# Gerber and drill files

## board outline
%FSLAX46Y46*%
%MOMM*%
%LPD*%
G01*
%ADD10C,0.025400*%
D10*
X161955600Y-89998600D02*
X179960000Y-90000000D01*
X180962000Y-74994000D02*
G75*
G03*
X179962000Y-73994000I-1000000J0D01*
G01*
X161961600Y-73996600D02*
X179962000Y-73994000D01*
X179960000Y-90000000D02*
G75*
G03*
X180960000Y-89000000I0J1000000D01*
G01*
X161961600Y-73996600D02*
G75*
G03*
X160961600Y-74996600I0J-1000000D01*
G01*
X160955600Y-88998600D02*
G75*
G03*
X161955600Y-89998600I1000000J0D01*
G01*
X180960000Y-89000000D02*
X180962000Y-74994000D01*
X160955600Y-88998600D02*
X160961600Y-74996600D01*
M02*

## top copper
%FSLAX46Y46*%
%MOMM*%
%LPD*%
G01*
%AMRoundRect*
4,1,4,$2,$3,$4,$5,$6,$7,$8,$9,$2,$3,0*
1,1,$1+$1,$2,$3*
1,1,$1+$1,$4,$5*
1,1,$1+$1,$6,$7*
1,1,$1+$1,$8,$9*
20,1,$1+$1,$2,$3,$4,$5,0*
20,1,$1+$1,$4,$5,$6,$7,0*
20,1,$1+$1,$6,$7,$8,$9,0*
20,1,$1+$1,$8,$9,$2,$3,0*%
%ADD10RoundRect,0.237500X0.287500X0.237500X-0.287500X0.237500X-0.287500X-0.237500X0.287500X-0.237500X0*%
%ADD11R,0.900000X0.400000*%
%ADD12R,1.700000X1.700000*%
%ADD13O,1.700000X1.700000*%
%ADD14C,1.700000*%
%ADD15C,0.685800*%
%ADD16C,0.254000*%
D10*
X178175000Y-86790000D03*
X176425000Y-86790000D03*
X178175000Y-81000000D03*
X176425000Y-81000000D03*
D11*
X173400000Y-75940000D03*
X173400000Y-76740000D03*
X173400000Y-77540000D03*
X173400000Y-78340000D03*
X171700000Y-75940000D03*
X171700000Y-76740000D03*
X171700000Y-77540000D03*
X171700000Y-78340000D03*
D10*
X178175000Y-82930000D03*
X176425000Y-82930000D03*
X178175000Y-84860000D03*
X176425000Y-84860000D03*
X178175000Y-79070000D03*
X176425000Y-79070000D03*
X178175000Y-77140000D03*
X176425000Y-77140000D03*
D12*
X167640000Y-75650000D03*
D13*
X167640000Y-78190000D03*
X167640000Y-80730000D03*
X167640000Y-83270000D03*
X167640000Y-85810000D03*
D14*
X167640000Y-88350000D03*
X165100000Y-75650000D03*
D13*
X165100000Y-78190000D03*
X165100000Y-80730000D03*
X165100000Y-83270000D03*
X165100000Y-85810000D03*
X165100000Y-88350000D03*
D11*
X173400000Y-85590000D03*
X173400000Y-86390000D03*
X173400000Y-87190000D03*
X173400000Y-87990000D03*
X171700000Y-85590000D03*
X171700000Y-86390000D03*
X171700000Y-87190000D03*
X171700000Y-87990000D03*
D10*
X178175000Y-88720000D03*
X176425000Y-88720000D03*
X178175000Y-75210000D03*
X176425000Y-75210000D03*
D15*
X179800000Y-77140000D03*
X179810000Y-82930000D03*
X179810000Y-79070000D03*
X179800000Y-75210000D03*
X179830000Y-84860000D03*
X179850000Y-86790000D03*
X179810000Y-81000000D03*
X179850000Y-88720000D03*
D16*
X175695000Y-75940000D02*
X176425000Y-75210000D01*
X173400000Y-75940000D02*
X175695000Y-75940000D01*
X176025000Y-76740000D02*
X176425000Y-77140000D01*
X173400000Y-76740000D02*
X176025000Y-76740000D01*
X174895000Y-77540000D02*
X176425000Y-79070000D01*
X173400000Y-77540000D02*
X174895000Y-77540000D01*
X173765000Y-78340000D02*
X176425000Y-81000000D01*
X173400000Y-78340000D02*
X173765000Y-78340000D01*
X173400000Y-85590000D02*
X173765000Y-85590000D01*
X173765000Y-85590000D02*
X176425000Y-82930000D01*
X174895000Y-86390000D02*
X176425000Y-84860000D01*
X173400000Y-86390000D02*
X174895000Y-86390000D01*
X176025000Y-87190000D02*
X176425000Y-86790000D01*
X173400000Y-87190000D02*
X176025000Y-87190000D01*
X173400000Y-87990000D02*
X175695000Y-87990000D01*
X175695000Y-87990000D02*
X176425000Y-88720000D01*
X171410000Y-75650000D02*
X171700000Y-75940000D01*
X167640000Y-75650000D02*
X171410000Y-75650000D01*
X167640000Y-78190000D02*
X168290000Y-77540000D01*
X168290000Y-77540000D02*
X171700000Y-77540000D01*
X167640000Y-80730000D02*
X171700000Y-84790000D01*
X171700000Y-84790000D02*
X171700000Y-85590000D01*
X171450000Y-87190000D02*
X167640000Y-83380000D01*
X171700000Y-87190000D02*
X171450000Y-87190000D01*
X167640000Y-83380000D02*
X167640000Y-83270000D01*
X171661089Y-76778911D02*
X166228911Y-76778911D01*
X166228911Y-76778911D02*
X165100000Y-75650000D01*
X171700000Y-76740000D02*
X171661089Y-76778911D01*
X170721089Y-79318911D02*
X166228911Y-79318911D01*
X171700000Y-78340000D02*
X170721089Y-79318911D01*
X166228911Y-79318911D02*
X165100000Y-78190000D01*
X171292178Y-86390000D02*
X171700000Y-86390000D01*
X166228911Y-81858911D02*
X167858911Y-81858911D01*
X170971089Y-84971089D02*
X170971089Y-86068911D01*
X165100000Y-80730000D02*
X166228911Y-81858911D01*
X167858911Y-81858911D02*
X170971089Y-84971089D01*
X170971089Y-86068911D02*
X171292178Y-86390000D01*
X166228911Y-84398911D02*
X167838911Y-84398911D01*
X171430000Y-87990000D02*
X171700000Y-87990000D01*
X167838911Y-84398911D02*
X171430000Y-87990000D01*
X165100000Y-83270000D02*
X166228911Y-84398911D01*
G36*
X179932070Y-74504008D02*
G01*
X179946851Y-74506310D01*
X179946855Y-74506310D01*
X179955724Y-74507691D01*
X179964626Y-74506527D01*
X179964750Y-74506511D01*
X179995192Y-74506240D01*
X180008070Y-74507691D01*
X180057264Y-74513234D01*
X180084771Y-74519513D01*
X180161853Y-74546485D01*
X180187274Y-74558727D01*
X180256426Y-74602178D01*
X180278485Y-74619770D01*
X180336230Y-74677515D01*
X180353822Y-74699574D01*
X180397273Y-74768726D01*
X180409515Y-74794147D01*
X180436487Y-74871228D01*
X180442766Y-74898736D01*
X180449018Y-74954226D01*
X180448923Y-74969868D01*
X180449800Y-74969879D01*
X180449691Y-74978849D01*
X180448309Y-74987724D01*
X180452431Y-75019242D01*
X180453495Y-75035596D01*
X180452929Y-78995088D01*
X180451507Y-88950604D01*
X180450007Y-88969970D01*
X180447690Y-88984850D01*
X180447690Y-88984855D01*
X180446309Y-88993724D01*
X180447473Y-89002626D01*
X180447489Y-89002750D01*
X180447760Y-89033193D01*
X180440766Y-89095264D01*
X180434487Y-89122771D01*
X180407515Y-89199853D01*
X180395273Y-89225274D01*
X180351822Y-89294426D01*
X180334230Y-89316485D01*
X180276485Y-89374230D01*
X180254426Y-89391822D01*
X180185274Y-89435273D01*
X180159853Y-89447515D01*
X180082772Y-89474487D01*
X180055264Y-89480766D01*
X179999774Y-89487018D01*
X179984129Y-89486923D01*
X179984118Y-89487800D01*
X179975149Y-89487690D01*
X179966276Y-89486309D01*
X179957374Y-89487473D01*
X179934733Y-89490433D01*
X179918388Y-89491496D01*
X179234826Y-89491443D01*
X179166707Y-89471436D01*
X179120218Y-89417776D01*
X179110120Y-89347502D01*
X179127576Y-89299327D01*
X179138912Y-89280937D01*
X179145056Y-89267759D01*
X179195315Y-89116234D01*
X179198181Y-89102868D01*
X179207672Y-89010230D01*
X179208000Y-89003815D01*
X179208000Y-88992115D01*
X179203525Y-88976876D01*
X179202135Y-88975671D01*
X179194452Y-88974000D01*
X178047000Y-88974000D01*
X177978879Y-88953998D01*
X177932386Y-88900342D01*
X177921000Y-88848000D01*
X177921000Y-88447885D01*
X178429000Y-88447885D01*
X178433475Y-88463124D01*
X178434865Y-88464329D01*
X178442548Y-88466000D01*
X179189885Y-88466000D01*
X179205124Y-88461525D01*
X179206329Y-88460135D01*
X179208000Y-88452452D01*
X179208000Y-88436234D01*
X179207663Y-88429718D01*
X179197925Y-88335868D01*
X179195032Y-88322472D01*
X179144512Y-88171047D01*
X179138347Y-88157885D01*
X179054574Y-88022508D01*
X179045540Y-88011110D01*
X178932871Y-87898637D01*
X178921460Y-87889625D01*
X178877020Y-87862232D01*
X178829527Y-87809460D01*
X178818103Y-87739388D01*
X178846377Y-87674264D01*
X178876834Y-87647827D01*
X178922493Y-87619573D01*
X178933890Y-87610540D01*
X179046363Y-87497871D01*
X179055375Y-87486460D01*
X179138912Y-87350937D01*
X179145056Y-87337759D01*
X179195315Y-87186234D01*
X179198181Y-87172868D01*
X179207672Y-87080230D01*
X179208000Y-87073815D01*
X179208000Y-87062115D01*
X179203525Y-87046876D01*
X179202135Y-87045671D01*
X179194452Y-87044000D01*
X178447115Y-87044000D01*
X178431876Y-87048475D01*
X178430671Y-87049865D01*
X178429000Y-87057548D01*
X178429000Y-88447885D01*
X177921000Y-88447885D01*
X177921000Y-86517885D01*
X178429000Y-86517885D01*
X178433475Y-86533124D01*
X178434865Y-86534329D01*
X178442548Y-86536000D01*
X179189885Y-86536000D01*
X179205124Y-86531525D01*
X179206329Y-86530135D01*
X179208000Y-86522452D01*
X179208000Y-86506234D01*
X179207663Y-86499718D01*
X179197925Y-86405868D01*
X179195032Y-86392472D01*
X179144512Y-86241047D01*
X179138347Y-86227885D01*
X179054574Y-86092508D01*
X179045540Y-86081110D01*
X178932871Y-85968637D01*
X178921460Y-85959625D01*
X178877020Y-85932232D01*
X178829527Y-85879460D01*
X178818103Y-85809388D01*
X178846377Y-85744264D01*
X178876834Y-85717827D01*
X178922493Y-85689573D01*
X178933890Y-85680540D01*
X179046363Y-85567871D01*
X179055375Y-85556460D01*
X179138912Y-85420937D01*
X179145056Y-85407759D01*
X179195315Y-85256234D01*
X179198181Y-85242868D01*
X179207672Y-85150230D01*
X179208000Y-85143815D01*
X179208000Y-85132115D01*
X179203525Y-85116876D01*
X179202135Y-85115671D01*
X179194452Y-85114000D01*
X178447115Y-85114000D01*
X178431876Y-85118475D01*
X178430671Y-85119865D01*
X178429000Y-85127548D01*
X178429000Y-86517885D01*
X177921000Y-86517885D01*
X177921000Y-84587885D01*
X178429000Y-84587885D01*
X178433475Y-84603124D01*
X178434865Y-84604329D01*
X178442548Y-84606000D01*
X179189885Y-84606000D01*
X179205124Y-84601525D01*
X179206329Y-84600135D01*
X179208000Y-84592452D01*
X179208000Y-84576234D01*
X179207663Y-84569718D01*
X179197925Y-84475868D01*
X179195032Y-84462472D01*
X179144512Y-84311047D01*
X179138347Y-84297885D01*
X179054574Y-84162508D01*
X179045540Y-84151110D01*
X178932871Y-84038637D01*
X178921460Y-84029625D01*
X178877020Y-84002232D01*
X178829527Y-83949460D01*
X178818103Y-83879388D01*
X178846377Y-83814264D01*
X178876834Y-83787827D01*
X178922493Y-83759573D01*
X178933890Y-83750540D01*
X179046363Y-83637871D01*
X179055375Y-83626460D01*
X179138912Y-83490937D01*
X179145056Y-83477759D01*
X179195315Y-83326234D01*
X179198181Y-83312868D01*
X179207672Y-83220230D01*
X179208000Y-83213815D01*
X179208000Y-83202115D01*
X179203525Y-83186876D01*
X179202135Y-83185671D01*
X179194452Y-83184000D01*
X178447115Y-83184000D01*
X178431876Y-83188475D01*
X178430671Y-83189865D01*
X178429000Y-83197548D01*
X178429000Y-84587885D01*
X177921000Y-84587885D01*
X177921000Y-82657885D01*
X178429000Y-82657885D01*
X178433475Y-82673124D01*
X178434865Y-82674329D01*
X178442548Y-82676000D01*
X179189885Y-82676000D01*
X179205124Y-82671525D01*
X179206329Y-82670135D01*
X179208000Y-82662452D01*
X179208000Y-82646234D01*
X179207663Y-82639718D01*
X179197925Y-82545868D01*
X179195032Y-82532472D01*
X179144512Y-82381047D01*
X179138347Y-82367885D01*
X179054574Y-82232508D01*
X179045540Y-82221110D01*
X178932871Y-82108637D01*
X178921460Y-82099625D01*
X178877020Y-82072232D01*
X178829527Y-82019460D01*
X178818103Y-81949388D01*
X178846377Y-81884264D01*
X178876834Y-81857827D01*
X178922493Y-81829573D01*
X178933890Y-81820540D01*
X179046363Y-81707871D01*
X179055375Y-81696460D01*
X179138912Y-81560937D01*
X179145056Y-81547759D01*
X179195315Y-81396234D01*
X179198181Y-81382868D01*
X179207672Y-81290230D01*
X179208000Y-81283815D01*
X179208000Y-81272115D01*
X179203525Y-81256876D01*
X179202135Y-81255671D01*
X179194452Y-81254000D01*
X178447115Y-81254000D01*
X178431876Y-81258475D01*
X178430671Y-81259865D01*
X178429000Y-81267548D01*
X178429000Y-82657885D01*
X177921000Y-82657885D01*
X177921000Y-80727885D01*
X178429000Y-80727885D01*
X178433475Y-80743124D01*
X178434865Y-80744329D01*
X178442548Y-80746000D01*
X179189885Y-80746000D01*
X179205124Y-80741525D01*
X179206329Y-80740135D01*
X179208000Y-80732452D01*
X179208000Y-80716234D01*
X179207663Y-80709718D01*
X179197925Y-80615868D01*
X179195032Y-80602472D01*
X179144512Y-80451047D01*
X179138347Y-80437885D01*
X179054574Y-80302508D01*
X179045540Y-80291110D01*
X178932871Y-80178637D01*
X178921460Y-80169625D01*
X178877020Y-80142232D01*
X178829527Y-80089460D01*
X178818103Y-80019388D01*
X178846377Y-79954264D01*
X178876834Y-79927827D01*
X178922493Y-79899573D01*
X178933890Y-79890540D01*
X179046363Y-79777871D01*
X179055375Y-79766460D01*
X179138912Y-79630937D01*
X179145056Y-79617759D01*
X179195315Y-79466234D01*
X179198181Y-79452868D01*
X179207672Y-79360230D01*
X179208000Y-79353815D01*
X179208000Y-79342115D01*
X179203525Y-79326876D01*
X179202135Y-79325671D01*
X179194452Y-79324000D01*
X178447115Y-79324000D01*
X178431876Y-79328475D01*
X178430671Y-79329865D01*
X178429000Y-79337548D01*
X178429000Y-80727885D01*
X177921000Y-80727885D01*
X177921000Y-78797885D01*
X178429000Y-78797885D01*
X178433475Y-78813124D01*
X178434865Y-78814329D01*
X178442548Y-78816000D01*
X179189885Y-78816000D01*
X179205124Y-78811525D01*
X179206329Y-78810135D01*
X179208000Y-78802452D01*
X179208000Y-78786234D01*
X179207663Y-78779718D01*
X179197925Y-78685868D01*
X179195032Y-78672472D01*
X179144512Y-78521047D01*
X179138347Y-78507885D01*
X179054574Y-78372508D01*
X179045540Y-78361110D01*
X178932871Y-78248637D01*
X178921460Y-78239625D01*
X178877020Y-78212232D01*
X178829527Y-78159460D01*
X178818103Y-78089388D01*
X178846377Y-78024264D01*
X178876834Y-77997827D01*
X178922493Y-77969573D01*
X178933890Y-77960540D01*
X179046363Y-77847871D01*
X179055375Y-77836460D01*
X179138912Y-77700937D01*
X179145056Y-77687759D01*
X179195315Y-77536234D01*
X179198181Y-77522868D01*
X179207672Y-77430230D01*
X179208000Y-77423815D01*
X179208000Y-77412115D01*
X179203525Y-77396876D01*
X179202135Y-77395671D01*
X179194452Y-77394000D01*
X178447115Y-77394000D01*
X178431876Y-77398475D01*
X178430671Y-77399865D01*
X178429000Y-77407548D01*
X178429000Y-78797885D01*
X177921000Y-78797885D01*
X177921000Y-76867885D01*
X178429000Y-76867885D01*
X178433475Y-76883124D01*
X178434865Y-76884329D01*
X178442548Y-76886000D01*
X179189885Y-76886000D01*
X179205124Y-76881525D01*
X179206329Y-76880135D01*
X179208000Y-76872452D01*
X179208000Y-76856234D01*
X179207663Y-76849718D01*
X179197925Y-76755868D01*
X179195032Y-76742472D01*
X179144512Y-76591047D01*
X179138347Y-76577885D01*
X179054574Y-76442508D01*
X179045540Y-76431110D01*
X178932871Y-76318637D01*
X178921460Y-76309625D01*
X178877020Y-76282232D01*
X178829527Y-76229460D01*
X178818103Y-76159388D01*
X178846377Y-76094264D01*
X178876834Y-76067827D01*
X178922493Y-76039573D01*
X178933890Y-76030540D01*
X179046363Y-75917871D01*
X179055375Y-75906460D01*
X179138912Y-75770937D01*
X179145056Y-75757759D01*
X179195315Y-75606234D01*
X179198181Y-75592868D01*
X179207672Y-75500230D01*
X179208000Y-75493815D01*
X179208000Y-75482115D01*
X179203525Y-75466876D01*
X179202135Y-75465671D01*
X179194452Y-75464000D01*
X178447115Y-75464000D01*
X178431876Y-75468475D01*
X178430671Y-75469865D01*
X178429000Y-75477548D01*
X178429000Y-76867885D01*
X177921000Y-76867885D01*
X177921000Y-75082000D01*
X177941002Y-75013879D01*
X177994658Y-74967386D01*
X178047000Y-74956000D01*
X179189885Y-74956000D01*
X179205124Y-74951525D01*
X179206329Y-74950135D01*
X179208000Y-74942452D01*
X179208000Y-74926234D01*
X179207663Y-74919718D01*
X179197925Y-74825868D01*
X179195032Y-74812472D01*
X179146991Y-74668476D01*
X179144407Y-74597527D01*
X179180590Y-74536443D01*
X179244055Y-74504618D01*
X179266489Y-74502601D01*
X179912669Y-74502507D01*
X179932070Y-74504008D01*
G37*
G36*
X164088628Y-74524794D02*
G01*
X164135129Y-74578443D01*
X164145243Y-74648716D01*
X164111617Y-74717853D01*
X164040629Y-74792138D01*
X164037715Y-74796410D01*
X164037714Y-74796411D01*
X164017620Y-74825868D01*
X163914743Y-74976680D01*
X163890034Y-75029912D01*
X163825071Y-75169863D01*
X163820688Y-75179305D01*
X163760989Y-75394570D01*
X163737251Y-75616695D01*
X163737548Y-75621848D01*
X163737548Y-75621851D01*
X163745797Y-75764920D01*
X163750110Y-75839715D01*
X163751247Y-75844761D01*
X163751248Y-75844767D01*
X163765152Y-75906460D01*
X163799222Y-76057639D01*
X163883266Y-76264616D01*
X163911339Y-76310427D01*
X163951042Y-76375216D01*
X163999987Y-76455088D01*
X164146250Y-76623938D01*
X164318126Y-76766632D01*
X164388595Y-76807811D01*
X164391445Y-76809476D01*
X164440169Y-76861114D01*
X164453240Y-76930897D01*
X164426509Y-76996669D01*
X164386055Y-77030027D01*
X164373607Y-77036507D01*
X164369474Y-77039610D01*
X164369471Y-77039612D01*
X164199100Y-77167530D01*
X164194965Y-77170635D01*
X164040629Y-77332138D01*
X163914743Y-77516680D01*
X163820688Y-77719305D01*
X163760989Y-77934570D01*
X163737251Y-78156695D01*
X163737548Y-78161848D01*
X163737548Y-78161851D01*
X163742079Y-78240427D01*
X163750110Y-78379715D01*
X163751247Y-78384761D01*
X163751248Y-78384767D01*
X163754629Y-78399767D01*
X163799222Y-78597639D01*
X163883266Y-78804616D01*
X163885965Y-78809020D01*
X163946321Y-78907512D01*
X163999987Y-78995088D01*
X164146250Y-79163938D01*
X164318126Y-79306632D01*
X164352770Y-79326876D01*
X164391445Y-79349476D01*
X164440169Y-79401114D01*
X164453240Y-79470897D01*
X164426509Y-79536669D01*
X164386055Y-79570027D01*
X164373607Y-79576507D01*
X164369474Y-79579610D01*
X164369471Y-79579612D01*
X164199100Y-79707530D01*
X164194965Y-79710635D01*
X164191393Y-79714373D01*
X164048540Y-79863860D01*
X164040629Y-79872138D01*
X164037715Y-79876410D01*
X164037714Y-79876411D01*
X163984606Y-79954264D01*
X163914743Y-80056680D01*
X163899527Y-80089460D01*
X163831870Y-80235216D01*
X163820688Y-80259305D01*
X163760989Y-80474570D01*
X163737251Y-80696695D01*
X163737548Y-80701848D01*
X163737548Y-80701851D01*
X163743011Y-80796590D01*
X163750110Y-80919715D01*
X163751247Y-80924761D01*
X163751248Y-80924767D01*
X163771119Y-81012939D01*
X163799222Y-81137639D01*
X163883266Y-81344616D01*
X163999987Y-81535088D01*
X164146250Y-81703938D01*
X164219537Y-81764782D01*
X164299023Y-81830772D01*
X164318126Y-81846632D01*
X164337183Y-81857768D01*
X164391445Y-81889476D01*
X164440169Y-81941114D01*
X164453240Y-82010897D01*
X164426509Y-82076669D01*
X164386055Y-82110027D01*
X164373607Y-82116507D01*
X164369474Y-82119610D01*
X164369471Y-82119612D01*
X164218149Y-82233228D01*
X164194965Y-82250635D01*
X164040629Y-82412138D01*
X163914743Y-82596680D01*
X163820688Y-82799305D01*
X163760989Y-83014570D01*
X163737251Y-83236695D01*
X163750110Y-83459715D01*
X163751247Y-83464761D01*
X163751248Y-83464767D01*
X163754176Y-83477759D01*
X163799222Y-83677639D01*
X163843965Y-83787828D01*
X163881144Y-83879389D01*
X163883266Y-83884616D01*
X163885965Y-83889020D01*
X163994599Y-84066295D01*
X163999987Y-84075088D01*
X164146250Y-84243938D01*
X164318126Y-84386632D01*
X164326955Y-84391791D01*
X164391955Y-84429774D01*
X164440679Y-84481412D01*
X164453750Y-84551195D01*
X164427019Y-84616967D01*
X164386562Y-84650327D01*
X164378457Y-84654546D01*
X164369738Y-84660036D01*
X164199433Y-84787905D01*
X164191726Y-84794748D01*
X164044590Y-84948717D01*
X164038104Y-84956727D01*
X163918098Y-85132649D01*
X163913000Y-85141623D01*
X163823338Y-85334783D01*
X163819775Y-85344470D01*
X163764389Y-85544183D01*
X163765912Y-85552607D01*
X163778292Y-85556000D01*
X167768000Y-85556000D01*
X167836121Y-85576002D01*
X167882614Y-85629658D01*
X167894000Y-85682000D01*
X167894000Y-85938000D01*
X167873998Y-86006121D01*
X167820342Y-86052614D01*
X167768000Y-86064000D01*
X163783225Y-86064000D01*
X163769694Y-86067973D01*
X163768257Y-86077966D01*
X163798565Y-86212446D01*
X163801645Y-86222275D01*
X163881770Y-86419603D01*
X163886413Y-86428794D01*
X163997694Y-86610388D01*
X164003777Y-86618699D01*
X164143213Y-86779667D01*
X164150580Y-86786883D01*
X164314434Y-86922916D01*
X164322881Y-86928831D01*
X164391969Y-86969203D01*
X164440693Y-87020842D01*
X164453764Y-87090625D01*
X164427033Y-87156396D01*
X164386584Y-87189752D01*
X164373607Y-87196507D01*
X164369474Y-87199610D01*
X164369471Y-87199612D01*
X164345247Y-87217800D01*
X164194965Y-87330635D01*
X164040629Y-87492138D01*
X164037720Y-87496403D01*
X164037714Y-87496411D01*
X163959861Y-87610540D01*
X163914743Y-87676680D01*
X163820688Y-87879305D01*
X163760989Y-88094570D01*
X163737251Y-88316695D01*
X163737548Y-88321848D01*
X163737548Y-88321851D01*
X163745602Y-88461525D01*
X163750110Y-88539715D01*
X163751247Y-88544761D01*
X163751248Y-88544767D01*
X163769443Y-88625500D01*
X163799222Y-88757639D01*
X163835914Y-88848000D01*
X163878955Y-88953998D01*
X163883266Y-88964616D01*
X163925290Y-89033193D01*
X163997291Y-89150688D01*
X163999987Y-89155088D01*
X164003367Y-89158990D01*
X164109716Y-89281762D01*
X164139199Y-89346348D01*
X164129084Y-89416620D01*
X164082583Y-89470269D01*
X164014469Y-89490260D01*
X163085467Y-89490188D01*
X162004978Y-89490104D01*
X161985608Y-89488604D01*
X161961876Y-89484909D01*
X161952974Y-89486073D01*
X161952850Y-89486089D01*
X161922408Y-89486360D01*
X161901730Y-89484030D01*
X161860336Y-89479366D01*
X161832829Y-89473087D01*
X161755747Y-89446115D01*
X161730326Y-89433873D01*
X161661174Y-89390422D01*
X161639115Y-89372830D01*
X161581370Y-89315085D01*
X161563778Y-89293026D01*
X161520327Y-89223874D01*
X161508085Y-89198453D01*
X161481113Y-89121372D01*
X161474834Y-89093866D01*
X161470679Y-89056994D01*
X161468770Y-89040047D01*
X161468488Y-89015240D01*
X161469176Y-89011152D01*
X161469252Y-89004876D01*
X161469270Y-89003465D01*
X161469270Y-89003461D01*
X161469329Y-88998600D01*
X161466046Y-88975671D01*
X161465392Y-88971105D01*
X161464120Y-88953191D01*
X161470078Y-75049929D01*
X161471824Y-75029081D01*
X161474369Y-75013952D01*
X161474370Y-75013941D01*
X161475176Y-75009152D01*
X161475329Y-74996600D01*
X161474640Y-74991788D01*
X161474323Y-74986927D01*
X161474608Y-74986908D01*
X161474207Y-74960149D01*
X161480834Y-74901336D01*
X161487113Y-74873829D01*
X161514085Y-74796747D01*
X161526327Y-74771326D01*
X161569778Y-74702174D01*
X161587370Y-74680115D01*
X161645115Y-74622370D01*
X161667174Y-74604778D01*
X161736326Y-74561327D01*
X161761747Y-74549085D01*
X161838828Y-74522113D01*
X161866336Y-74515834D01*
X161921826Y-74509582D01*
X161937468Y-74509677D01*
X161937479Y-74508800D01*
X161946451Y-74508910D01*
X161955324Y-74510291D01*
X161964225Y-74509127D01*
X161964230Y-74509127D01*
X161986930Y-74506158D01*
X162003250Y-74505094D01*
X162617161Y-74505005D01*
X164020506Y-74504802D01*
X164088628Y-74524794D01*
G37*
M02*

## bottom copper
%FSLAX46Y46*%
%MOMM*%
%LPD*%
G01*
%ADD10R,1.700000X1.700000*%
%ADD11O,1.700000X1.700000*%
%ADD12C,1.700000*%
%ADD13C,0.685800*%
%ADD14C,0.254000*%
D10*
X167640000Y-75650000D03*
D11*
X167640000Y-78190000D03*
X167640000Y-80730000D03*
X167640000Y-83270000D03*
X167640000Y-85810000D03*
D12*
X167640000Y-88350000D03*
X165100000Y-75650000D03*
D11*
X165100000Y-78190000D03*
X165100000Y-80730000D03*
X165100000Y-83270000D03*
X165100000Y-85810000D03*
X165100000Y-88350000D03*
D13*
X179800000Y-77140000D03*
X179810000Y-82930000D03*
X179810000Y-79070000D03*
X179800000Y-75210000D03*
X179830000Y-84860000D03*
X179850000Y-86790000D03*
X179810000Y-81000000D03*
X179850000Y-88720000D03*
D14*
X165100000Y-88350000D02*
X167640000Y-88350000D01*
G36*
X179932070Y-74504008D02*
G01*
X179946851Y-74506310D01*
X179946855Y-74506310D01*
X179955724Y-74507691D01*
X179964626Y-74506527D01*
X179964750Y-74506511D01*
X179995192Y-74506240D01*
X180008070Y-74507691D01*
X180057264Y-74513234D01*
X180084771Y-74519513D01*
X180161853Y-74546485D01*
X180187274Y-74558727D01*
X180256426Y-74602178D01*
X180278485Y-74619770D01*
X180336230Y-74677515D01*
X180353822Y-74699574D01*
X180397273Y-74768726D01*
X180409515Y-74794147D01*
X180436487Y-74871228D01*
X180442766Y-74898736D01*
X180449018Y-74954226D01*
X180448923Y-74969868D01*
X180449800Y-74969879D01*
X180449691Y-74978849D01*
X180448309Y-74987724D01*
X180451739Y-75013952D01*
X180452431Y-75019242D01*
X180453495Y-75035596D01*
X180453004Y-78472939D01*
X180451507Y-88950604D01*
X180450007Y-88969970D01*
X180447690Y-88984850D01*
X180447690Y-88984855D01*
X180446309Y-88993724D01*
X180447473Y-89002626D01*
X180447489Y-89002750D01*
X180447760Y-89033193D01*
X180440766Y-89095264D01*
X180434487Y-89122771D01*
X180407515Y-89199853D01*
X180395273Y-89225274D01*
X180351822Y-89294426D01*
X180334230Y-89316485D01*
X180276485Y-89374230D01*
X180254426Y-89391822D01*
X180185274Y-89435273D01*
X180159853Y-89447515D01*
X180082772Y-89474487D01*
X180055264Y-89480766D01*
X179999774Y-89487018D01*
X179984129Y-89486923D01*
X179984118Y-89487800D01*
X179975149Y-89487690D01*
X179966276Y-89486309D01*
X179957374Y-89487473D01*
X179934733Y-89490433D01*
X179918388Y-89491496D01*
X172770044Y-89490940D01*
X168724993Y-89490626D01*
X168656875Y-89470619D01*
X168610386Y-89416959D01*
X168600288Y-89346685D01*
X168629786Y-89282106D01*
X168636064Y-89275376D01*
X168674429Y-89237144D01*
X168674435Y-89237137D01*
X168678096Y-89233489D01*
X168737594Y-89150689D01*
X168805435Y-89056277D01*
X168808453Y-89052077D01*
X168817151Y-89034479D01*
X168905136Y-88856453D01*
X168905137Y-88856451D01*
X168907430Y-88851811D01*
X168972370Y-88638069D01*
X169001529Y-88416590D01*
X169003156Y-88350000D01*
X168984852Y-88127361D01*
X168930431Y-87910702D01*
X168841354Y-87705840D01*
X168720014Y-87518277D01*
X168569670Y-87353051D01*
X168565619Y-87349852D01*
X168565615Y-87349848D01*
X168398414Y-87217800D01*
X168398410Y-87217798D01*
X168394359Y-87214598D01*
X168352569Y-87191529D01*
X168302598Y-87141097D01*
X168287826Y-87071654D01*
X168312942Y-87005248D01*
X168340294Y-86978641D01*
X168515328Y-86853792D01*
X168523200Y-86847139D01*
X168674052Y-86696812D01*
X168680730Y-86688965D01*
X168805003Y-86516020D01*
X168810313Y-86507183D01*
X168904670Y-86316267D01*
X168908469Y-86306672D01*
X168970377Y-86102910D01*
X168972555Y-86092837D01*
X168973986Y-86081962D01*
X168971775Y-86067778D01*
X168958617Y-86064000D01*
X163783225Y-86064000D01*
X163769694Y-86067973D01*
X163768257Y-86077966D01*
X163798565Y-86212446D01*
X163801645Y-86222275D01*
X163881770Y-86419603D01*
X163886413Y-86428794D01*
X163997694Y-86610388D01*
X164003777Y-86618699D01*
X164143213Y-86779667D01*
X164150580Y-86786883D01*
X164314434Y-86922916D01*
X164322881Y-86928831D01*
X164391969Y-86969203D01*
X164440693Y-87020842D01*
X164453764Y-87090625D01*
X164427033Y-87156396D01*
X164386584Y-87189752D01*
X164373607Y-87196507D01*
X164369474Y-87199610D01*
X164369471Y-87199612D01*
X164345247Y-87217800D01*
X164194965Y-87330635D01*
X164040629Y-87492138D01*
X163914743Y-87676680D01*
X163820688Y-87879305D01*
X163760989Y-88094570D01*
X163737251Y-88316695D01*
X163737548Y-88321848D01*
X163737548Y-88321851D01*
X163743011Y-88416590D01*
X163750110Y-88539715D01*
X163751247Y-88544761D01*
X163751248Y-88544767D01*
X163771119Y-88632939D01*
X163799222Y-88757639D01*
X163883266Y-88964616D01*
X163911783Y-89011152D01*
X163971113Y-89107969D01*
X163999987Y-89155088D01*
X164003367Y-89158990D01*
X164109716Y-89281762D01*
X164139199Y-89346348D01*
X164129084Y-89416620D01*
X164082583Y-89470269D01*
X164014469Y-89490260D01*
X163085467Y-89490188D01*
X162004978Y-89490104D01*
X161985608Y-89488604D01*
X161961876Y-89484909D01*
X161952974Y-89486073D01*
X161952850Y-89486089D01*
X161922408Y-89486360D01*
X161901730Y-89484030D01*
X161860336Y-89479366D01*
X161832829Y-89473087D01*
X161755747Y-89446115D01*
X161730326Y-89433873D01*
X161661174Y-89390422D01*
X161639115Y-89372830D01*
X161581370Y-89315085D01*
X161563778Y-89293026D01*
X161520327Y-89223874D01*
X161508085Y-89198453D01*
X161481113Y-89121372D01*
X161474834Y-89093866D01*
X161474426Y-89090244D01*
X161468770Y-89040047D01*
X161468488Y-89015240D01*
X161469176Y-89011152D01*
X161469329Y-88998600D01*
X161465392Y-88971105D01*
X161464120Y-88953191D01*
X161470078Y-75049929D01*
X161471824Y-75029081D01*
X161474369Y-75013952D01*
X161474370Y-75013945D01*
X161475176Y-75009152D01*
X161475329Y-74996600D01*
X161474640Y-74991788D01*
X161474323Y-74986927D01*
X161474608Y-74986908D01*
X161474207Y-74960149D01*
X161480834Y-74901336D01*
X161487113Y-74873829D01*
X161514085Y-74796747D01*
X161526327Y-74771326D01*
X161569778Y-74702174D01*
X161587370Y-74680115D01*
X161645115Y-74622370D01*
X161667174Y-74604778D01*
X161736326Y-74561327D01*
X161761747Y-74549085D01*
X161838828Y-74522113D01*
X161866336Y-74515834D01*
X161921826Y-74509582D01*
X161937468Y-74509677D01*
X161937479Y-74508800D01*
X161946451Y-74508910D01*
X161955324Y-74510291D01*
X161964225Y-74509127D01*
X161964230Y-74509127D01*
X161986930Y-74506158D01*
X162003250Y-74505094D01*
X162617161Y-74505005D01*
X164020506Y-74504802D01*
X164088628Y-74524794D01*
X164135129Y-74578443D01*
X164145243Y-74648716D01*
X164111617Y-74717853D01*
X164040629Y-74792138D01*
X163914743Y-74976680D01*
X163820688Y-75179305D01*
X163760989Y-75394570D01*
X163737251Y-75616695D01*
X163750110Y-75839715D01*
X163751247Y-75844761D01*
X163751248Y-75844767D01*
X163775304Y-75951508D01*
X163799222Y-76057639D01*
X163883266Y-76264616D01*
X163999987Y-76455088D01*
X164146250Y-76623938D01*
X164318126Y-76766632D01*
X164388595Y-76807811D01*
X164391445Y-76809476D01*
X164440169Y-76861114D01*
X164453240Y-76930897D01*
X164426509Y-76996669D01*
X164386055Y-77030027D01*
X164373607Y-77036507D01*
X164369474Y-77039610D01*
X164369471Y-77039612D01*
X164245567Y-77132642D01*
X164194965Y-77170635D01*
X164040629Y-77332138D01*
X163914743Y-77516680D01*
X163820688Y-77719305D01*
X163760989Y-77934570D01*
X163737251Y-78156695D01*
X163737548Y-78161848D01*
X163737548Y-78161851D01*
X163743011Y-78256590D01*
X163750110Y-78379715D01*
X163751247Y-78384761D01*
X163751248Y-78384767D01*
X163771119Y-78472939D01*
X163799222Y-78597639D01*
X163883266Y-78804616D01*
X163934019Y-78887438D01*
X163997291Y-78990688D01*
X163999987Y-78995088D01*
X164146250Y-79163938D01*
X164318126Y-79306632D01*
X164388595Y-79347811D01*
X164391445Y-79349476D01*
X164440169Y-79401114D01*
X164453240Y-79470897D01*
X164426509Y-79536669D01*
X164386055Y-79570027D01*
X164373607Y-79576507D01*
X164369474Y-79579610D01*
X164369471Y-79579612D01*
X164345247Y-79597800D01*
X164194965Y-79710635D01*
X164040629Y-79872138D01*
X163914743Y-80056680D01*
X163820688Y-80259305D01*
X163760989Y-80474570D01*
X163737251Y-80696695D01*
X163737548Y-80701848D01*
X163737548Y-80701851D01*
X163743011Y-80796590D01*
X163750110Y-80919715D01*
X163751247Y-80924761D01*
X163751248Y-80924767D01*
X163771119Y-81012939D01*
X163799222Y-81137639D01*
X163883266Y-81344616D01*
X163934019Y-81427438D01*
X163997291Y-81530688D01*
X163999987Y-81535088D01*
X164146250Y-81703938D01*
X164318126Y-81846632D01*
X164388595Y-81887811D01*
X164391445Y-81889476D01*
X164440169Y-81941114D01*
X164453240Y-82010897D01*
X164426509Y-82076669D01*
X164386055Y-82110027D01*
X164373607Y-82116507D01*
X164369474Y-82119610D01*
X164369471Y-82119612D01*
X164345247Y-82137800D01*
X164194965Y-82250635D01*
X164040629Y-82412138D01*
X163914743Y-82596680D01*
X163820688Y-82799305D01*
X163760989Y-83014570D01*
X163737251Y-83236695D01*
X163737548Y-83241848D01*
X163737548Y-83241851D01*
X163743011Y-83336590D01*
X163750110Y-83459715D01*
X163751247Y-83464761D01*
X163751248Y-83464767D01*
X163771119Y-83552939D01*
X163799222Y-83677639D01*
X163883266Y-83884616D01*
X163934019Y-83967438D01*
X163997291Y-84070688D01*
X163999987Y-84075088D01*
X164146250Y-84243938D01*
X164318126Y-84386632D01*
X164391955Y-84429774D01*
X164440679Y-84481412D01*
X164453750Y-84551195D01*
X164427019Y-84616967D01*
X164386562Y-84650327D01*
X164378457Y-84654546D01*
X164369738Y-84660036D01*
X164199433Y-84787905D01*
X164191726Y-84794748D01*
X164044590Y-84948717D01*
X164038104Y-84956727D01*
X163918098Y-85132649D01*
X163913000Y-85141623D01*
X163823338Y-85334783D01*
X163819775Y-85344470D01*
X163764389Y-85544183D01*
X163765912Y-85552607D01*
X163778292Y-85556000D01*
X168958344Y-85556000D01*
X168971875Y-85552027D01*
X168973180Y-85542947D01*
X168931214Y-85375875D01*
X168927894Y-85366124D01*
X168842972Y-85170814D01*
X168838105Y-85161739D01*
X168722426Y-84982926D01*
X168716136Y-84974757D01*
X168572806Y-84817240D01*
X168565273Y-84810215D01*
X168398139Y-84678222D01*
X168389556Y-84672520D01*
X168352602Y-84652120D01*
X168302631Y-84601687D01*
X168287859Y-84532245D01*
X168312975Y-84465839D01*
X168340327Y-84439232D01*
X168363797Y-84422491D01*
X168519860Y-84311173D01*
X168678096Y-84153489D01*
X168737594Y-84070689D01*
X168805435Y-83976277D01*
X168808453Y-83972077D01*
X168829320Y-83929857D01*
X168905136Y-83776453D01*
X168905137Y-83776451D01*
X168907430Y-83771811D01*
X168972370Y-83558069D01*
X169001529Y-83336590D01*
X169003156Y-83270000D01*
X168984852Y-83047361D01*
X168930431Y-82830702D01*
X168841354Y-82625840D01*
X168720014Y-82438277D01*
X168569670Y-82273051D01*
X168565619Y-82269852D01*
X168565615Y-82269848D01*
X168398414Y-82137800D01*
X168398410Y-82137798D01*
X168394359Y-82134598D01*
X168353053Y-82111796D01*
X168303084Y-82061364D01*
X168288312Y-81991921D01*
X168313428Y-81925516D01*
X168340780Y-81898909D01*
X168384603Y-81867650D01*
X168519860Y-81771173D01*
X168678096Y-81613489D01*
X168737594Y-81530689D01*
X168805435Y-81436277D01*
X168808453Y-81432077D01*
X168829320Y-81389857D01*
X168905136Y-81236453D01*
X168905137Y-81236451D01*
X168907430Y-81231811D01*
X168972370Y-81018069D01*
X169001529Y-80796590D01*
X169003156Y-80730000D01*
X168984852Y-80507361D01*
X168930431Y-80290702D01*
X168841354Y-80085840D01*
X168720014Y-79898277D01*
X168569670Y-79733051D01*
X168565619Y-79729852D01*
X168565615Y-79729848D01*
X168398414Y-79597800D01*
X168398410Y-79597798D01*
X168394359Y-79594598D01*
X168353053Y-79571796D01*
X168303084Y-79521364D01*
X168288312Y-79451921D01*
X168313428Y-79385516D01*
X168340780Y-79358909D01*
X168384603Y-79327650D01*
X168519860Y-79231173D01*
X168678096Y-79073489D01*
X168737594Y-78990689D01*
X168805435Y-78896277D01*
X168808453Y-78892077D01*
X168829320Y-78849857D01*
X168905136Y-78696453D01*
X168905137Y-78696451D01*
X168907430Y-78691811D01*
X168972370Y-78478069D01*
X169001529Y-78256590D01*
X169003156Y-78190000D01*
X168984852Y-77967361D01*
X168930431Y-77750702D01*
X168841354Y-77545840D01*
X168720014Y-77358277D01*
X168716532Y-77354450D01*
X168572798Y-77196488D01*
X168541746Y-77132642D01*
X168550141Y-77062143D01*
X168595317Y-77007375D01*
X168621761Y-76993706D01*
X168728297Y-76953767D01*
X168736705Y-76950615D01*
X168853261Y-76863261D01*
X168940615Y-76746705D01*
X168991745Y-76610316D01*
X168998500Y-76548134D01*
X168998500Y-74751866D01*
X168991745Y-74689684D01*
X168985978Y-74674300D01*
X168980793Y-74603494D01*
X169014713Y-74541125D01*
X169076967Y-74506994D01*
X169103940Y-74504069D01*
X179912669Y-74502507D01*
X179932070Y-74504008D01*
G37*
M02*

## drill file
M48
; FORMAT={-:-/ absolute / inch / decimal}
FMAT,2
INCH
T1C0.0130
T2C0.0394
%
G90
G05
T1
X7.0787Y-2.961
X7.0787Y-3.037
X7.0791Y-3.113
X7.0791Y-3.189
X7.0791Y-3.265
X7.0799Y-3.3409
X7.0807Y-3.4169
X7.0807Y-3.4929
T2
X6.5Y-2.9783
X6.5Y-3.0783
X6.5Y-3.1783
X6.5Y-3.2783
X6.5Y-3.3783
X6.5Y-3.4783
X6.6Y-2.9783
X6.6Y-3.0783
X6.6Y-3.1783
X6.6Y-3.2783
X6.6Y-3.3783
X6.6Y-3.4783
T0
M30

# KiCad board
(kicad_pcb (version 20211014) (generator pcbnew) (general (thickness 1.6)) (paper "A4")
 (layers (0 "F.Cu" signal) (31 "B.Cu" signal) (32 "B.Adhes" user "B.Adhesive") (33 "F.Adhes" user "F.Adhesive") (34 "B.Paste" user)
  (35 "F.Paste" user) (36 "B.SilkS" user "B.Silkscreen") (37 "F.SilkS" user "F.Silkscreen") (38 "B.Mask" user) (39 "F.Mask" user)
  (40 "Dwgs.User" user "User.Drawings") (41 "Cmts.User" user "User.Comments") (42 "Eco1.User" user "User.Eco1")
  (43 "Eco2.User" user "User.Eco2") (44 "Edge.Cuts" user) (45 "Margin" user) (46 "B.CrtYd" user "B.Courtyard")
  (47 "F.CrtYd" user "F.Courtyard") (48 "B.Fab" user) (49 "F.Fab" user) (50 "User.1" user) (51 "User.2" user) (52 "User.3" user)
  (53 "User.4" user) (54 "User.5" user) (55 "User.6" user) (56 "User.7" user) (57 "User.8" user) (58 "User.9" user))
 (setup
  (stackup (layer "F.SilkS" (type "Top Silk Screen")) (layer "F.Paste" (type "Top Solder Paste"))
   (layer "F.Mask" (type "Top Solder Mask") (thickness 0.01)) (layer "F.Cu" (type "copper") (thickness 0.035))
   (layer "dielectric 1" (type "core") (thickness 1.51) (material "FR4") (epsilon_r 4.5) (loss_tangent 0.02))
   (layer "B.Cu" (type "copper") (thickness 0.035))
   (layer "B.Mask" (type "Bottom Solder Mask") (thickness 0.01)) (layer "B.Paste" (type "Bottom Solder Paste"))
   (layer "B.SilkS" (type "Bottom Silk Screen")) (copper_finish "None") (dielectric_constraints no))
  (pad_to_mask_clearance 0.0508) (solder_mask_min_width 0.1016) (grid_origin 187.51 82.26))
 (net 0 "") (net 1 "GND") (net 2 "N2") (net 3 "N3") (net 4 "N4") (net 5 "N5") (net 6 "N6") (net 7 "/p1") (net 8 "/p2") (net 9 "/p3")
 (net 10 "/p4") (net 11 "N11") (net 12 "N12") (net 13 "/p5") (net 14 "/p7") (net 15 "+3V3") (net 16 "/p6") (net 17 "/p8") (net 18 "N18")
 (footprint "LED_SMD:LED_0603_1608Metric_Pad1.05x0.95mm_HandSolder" (layer "F.Cu") (at 177.3 86.79 180)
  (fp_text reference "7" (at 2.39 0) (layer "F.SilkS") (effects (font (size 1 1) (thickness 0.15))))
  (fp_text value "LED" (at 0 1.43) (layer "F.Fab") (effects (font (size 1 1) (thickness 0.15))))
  (pad "1" smd roundrect (at -0.875 0 180) (size 1.05 0.95) (layers "F.Cu" "F.Paste" "F.Mask") (roundrect_rratio 0.25) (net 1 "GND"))
  (pad "2" smd roundrect (at 0.875 0 180) (size 1.05 0.95) (layers "F.Cu" "F.Paste" "F.Mask") (roundrect_rratio 0.25) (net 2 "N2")))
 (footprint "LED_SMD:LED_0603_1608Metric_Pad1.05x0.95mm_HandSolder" (layer "F.Cu") (at 177.3 81 180)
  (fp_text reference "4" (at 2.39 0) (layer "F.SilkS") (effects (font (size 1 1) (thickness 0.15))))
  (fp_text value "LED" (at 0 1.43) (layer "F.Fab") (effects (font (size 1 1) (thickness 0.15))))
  (pad "1" smd roundrect (at -0.875 0 180) (size 1.05 0.95) (layers "F.Cu" "F.Paste" "F.Mask") (roundrect_rratio 0.25) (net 1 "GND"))
  (pad "2" smd roundrect (at 0.875 0 180) (size 1.05 0.95) (layers "F.Cu" "F.Paste" "F.Mask") (roundrect_rratio 0.25) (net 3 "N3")))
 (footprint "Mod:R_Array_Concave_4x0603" (layer "F.Cu") (at 172.55 77.14 180)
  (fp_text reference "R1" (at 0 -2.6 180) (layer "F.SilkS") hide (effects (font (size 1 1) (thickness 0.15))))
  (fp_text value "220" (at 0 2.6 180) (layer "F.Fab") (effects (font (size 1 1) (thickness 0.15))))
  (pad "1" smd rect (at -0.85 1.2 180) (size 0.9 0.4) (layers "F.Cu" "F.Paste" "F.Mask") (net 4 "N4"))
  (pad "2" smd rect (at -0.85 0.4 180) (size 0.9 0.4) (layers "F.Cu" "F.Paste" "F.Mask") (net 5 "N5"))
  (pad "3" smd rect (at -0.85 -0.4 180) (size 0.9 0.4) (layers "F.Cu" "F.Paste" "F.Mask") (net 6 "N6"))
  (pad "4" smd rect (at -0.85 -1.2 180) (size 0.9 0.4) (layers "F.Cu" "F.Paste" "F.Mask") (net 3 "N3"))
  (pad "5" smd rect (at 0.85 1.2 180) (size 0.9 0.4) (layers "F.Cu" "F.Paste" "F.Mask") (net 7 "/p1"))
  (pad "6" smd rect (at 0.85 0.4 180) (size 0.9 0.4) (layers "F.Cu" "F.Paste" "F.Mask") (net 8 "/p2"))
  (pad "7" smd rect (at 0.85 -0.4 180) (size 0.9 0.4) (layers "F.Cu" "F.Paste" "F.Mask") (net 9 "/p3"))
  (pad "8" smd rect (at 0.85 -1.2 180) (size 0.9 0.4) (layers "F.Cu" "F.Paste" "F.Mask") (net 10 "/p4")))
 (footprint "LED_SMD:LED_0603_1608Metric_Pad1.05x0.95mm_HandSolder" (layer "F.Cu") (at 177.3 82.93 180)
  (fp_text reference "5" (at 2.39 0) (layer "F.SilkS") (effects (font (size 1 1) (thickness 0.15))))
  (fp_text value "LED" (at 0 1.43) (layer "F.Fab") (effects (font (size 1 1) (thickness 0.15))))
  (pad "1" smd roundrect (at -0.875 0 180) (size 1.05 0.95) (layers "F.Cu" "F.Paste" "F.Mask") (roundrect_rratio 0.25) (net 1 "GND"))
  (pad "2" smd roundrect (at 0.875 0 180) (size 1.05 0.95) (layers "F.Cu" "F.Paste" "F.Mask") (roundrect_rratio 0.25) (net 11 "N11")))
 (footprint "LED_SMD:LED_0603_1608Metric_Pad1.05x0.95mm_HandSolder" (layer "F.Cu") (at 177.3 84.86 180)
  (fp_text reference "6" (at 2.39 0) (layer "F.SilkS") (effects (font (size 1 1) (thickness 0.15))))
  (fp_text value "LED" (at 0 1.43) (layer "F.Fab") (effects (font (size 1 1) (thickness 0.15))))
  (pad "1" smd roundrect (at -0.875 0 180) (size 1.05 0.95) (layers "F.Cu" "F.Paste" "F.Mask") (roundrect_rratio 0.25) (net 1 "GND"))
  (pad "2" smd roundrect (at 0.875 0 180) (size 1.05 0.95) (layers "F.Cu" "F.Paste" "F.Mask") (roundrect_rratio 0.25) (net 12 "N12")))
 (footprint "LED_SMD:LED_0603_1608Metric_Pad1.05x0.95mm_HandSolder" (layer "F.Cu") (at 177.3 79.07 180)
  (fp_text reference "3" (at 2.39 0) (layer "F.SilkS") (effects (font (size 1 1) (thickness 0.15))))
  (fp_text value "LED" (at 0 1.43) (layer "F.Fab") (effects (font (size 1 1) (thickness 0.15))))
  (pad "1" smd roundrect (at -0.875 0 180) (size 1.05 0.95) (layers "F.Cu" "F.Paste" "F.Mask") (roundrect_rratio 0.25) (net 1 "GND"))
  (pad "2" smd roundrect (at 0.875 0 180) (size 1.05 0.95) (layers "F.Cu" "F.Paste" "F.Mask") (roundrect_rratio 0.25) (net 6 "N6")))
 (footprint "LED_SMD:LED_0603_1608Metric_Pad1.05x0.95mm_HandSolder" (layer "F.Cu") (at 177.3 77.14 180)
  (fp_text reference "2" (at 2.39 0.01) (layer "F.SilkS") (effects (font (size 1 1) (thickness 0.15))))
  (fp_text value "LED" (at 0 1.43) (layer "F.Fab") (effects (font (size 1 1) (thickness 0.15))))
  (pad "1" smd roundrect (at -0.875 0 180) (size 1.05 0.95) (layers "F.Cu" "F.Paste" "F.Mask") (roundrect_rratio 0.25) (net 1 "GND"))
  (pad "2" smd roundrect (at 0.875 0 180) (size 1.05 0.95) (layers "F.Cu" "F.Paste" "F.Mask") (roundrect_rratio 0.25) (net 5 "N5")))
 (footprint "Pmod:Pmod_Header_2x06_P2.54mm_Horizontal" (layer "F.Cu") (at 167.64 88.35 180)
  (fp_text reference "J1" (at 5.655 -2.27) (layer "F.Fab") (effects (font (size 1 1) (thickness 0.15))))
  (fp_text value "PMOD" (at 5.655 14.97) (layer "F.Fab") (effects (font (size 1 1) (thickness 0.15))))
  (pad "1" thru_hole rect (at 0 12.7 180) (size 1.7 1.7) (drill 1) (layers *.Cu *.Mask) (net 7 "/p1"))
  (pad "2" thru_hole oval (at 0 10.16 180) (size 1.7 1.7) (drill 1) (layers *.Cu *.Mask) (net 9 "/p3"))
  (pad "3" thru_hole oval (at 0 7.62 180) (size 1.7 1.7) (drill 1) (layers *.Cu *.Mask) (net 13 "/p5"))
  (pad "4" thru_hole oval (at 0 5.08 180) (size 1.7 1.7) (drill 1) (layers *.Cu *.Mask) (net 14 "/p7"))
  (pad "5" thru_hole oval (at 0 2.54 180) (size 1.7 1.7) (drill 1) (layers *.Cu *.Mask) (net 1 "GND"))
  (pad "6" thru_hole circle (at 0 0 180) (size 1.7 1.7) (drill 1) (layers *.Cu *.Mask) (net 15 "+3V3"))
  (pad "7" thru_hole circle (at 2.54 12.7 180) (size 1.7 1.7) (drill 1) (layers *.Cu *.Mask) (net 8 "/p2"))
  (pad "8" thru_hole oval (at 2.54 10.16 180) (size 1.7 1.7) (drill 1) (layers *.Cu *.Mask) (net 10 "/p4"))
  (pad "9" thru_hole oval (at 2.54 7.62 180) (size 1.7 1.7) (drill 1) (layers *.Cu *.Mask) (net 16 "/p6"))
  (pad "10" thru_hole oval (at 2.54 5.08 180) (size 1.7 1.7) (drill 1) (layers *.Cu *.Mask) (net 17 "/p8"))
  (pad "11" thru_hole oval (at 2.54 2.54 180) (size 1.7 1.7) (drill 1) (layers *.Cu *.Mask) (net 1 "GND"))
  (pad "12" thru_hole oval (at 2.54 0 180) (size 1.7 1.7) (drill 1) (layers *.Cu *.Mask) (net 15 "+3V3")))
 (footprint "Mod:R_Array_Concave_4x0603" (layer "F.Cu") (at 172.55 86.79 180)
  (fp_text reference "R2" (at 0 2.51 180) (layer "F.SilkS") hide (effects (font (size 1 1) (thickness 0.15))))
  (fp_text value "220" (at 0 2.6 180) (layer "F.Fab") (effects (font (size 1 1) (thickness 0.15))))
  (pad "1" smd rect (at -0.85 1.2 180) (size 0.9 0.4) (layers "F.Cu" "F.Paste" "F.Mask") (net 11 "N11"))
  (pad "2" smd rect (at -0.85 0.4 180) (size 0.9 0.4) (layers "F.Cu" "F.Paste" "F.Mask") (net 12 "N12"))
  (pad "3" smd rect (at -0.85 -0.4 180) (size 0.9 0.4) (layers "F.Cu" "F.Paste" "F.Mask") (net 2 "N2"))
  (pad "4" smd rect (at -0.85 -1.2 180) (size 0.9 0.4) (layers "F.Cu" "F.Paste" "F.Mask") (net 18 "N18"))
  (pad "5" smd rect (at 0.85 1.2 180) (size 0.9 0.4) (layers "F.Cu" "F.Paste" "F.Mask") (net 13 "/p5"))
  (pad "6" smd rect (at 0.85 0.4 180) (size 0.9 0.4) (layers "F.Cu" "F.Paste" "F.Mask") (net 16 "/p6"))
  (pad "7" smd rect (at 0.85 -0.4 180) (size 0.9 0.4) (layers "F.Cu" "F.Paste" "F.Mask") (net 14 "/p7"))
  (pad "8" smd rect (at 0.85 -1.2 180) (size 0.9 0.4) (layers "F.Cu" "F.Paste" "F.Mask") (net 17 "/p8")))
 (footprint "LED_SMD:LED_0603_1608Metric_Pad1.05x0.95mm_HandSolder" (layer "F.Cu") (at 177.3 88.72 180)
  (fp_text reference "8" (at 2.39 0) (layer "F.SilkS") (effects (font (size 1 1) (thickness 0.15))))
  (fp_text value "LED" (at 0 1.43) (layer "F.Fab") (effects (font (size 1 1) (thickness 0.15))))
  (pad "1" smd roundrect (at -0.875 0 180) (size 1.05 0.95) (layers "F.Cu" "F.Paste" "F.Mask") (roundrect_rratio 0.25) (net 1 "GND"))
  (pad "2" smd roundrect (at 0.875 0 180) (size 1.05 0.95) (layers "F.Cu" "F.Paste" "F.Mask") (roundrect_rratio 0.25) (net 18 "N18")))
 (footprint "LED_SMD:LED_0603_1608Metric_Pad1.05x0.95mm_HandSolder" (layer "F.Cu") (at 177.3 75.21 180)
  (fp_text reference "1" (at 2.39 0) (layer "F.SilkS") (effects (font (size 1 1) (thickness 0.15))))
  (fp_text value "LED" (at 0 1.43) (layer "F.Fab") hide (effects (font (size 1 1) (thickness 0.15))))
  (pad "1" smd roundrect (at -0.875 0 180) (size 1.05 0.95) (layers "F.Cu" "F.Paste" "F.Mask") (roundrect_rratio 0.25) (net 1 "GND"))
  (pad "2" smd roundrect (at 0.875 0 180) (size 1.05 0.95) (layers "F.Cu" "F.Paste" "F.Mask") (roundrect_rratio 0.25) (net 4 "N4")))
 (gr_line (start 161.9556 89.9986) (end 179.96 90) (layer "Edge.Cuts") (width 0.0254))
 (gr_arc (start 179.962 73.994) (mid 180.669112 74.286888) (end 180.962 74.994) (layer "Edge.Cuts") (width 0.0254))
 (gr_line (start 161.9616 73.9966) (end 179.962 73.994) (layer "Edge.Cuts") (width 0.0254))
 (gr_arc (start 180.96 89) (mid 180.667109 89.707109) (end 179.96 90) (layer "Edge.Cuts") (width 0.0254))
 (gr_arc (start 160.9616 74.9966) (mid 161.254495 74.289495) (end 161.9616 73.9966) (layer "Edge.Cuts") (width 0.0254))
 (gr_arc (start 161.9556 89.9986) (mid 161.248498 89.705702) (end 160.9556 88.9986) (layer "Edge.Cuts") (width 0.0254))
 (gr_line (start 180.96 89) (end 180.962 74.994) (layer "Edge.Cuts") (width 0.0254))
 (gr_line (start 160.9556 88.9986) (end 160.9616 74.9966) (layer "Edge.Cuts") (width 0.0254))
 (via (at 179.8 77.14) (size 0.6858) (drill 0.3302) (layers "F.Cu" "B.Cu") (free) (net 1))
 (via (at 179.81 82.93) (size 0.6858) (drill 0.3302) (layers "F.Cu" "B.Cu") (free) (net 1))
 (via (at 179.81 79.07) (size 0.6858) (drill 0.3302) (layers "F.Cu" "B.Cu") (free) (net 1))
 (via (at 179.8 75.21) (size 0.6858) (drill 0.3302) (layers "F.Cu" "B.Cu") (free) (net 1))
 (via (at 179.83 84.86) (size 0.6858) (drill 0.3302) (layers "F.Cu" "B.Cu") (free) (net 1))
 (via (at 179.85 86.79) (size 0.6858) (drill 0.3302) (layers "F.Cu" "B.Cu") (free) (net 1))
 (via (at 179.81 81) (size 0.6858) (drill 0.3302) (layers "F.Cu" "B.Cu") (free) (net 1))
 (via (at 179.85 88.72) (size 0.6858) (drill 0.3302) (layers "F.Cu" "B.Cu") (free) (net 1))
 (segment (start 175.695 75.94) (end 176.425 75.21) (width 0.254) (layer "F.Cu") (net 4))
 (segment (start 173.4 75.94) (end 175.695 75.94) (width 0.254) (layer "F.Cu") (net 4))
 (segment (start 176.025 76.74) (end 176.425 77.14) (width 0.254) (layer "F.Cu") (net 5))
 (segment (start 173.4 76.74) (end 176.025 76.74) (width 0.254) (layer "F.Cu") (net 5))
 (segment (start 174.895 77.54) (end 176.425 79.07) (width 0.254) (layer "F.Cu") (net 6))
 (segment (start 173.4 77.54) (end 174.895 77.54) (width 0.254) (layer "F.Cu") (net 6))
 (segment (start 173.765 78.34) (end 176.425 81) (width 0.254) (layer "F.Cu") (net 3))
 (segment (start 173.4 78.34) (end 173.765 78.34) (width 0.254) (layer "F.Cu") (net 3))
 (segment (start 173.4 85.59) (end 173.765 85.59) (width 0.254) (layer "F.Cu") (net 11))
 (segment (start 173.765 85.59) (end 176.425 82.93) (width 0.254) (layer "F.Cu") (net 11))
 (segment (start 174.895 86.39) (end 176.425 84.86) (width 0.254) (layer "F.Cu") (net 12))
 (segment (start 173.4 86.39) (end 174.895 86.39) (width 0.254) (layer "F.Cu") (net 12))
 (segment (start 176.025 87.19) (end 176.425 86.79) (width 0.254) (layer "F.Cu") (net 2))
 (segment (start 173.4 87.19) (end 176.025 87.19) (width 0.254) (layer "F.Cu") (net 2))
 (segment (start 173.4 87.99) (end 175.695 87.99) (width 0.254) (layer "F.Cu") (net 18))
 (segment (start 175.695 87.99) (end 176.425 88.72) (width 0.254) (layer "F.Cu") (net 18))
 (segment (start 171.41 75.65) (end 171.7 75.94) (width 0.254) (layer "F.Cu") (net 7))
 (segment (start 167.64 75.65) (end 171.41 75.65) (width 0.254) (layer "F.Cu") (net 7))
 (segment (start 167.64 78.19) (end 168.29 77.54) (width 0.254) (layer "F.Cu") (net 9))
 (segment (start 168.29 77.54) (end 171.7 77.54) (width 0.254) (layer "F.Cu") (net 9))
 (segment (start 167.64 80.73) (end 171.7 84.79) (width 0.254) (layer "F.Cu") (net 13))
 (segment (start 171.7 84.79) (end 171.7 85.59) (width 0.254) (layer "F.Cu") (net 13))
 (segment (start 171.45 87.19) (end 167.64 83.38) (width 0.254) (layer "F.Cu") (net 14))
 (segment (start 171.7 87.19) (end 171.45 87.19) (width 0.254) (layer "F.Cu") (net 14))
 (segment (start 167.64 83.38) (end 167.64 83.27) (width 0.254) (layer "F.Cu") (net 14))
 (segment (start 165.1 88.35) (end 167.64 88.35) (width 0.254) (layer "B.Cu") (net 15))
 (segment (start 171.661089 76.778911) (end 166.228911 76.778911) (width 0.254) (layer "F.Cu") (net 8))
 (segment (start 166.228911 76.778911) (end 165.1 75.65) (width 0.254) (layer "F.Cu") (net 8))
 (segment (start 171.7 76.74) (end 171.661089 76.778911) (width 0.254) (layer "F.Cu") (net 8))
 (segment (start 170.721089 79.318911) (end 166.228911 79.318911) (width 0.254) (layer "F.Cu") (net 10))
 (segment (start 171.7 78.34) (end 170.721089 79.318911) (width 0.254) (layer "F.Cu") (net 10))
 (segment (start 166.228911 79.318911) (end 165.1 78.19) (width 0.254) (layer "F.Cu") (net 10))
 (segment (start 171.292178 86.39) (end 171.7 86.39) (width 0.254) (layer "F.Cu") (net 16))
 (segment (start 166.228911 81.858911) (end 167.858911 81.858911) (width 0.254) (layer "F.Cu") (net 16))
 (segment (start 170.971089 84.971089) (end 170.971089 86.068911) (width 0.254) (layer "F.Cu") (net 16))
 (segment (start 165.1 80.73) (end 166.228911 81.858911) (width 0.254) (layer "F.Cu") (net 16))
 (segment (start 167.858911 81.858911) (end 170.971089 84.971089) (width 0.254) (layer "F.Cu") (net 16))
 (segment (start 170.971089 86.068911) (end 171.292178 86.39) (width 0.254) (layer "F.Cu") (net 16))
 (segment (start 166.228911 84.398911) (end 167.838911 84.398911) (width 0.254) (layer "F.Cu") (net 17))
 (segment (start 171.43 87.99) (end 171.7 87.99) (width 0.254) (layer "F.Cu") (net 17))
 (segment (start 167.838911 84.398911) (end 171.43 87.99) (width 0.254) (layer "F.Cu") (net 17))
 (segment (start 165.1 83.27) (end 166.228911 84.398911) (width 0.254) (layer "F.Cu") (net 17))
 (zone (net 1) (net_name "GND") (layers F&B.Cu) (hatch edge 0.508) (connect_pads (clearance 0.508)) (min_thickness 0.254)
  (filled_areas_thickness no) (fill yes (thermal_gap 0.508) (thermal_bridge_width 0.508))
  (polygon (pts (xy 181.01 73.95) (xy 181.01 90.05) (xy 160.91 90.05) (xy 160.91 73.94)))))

